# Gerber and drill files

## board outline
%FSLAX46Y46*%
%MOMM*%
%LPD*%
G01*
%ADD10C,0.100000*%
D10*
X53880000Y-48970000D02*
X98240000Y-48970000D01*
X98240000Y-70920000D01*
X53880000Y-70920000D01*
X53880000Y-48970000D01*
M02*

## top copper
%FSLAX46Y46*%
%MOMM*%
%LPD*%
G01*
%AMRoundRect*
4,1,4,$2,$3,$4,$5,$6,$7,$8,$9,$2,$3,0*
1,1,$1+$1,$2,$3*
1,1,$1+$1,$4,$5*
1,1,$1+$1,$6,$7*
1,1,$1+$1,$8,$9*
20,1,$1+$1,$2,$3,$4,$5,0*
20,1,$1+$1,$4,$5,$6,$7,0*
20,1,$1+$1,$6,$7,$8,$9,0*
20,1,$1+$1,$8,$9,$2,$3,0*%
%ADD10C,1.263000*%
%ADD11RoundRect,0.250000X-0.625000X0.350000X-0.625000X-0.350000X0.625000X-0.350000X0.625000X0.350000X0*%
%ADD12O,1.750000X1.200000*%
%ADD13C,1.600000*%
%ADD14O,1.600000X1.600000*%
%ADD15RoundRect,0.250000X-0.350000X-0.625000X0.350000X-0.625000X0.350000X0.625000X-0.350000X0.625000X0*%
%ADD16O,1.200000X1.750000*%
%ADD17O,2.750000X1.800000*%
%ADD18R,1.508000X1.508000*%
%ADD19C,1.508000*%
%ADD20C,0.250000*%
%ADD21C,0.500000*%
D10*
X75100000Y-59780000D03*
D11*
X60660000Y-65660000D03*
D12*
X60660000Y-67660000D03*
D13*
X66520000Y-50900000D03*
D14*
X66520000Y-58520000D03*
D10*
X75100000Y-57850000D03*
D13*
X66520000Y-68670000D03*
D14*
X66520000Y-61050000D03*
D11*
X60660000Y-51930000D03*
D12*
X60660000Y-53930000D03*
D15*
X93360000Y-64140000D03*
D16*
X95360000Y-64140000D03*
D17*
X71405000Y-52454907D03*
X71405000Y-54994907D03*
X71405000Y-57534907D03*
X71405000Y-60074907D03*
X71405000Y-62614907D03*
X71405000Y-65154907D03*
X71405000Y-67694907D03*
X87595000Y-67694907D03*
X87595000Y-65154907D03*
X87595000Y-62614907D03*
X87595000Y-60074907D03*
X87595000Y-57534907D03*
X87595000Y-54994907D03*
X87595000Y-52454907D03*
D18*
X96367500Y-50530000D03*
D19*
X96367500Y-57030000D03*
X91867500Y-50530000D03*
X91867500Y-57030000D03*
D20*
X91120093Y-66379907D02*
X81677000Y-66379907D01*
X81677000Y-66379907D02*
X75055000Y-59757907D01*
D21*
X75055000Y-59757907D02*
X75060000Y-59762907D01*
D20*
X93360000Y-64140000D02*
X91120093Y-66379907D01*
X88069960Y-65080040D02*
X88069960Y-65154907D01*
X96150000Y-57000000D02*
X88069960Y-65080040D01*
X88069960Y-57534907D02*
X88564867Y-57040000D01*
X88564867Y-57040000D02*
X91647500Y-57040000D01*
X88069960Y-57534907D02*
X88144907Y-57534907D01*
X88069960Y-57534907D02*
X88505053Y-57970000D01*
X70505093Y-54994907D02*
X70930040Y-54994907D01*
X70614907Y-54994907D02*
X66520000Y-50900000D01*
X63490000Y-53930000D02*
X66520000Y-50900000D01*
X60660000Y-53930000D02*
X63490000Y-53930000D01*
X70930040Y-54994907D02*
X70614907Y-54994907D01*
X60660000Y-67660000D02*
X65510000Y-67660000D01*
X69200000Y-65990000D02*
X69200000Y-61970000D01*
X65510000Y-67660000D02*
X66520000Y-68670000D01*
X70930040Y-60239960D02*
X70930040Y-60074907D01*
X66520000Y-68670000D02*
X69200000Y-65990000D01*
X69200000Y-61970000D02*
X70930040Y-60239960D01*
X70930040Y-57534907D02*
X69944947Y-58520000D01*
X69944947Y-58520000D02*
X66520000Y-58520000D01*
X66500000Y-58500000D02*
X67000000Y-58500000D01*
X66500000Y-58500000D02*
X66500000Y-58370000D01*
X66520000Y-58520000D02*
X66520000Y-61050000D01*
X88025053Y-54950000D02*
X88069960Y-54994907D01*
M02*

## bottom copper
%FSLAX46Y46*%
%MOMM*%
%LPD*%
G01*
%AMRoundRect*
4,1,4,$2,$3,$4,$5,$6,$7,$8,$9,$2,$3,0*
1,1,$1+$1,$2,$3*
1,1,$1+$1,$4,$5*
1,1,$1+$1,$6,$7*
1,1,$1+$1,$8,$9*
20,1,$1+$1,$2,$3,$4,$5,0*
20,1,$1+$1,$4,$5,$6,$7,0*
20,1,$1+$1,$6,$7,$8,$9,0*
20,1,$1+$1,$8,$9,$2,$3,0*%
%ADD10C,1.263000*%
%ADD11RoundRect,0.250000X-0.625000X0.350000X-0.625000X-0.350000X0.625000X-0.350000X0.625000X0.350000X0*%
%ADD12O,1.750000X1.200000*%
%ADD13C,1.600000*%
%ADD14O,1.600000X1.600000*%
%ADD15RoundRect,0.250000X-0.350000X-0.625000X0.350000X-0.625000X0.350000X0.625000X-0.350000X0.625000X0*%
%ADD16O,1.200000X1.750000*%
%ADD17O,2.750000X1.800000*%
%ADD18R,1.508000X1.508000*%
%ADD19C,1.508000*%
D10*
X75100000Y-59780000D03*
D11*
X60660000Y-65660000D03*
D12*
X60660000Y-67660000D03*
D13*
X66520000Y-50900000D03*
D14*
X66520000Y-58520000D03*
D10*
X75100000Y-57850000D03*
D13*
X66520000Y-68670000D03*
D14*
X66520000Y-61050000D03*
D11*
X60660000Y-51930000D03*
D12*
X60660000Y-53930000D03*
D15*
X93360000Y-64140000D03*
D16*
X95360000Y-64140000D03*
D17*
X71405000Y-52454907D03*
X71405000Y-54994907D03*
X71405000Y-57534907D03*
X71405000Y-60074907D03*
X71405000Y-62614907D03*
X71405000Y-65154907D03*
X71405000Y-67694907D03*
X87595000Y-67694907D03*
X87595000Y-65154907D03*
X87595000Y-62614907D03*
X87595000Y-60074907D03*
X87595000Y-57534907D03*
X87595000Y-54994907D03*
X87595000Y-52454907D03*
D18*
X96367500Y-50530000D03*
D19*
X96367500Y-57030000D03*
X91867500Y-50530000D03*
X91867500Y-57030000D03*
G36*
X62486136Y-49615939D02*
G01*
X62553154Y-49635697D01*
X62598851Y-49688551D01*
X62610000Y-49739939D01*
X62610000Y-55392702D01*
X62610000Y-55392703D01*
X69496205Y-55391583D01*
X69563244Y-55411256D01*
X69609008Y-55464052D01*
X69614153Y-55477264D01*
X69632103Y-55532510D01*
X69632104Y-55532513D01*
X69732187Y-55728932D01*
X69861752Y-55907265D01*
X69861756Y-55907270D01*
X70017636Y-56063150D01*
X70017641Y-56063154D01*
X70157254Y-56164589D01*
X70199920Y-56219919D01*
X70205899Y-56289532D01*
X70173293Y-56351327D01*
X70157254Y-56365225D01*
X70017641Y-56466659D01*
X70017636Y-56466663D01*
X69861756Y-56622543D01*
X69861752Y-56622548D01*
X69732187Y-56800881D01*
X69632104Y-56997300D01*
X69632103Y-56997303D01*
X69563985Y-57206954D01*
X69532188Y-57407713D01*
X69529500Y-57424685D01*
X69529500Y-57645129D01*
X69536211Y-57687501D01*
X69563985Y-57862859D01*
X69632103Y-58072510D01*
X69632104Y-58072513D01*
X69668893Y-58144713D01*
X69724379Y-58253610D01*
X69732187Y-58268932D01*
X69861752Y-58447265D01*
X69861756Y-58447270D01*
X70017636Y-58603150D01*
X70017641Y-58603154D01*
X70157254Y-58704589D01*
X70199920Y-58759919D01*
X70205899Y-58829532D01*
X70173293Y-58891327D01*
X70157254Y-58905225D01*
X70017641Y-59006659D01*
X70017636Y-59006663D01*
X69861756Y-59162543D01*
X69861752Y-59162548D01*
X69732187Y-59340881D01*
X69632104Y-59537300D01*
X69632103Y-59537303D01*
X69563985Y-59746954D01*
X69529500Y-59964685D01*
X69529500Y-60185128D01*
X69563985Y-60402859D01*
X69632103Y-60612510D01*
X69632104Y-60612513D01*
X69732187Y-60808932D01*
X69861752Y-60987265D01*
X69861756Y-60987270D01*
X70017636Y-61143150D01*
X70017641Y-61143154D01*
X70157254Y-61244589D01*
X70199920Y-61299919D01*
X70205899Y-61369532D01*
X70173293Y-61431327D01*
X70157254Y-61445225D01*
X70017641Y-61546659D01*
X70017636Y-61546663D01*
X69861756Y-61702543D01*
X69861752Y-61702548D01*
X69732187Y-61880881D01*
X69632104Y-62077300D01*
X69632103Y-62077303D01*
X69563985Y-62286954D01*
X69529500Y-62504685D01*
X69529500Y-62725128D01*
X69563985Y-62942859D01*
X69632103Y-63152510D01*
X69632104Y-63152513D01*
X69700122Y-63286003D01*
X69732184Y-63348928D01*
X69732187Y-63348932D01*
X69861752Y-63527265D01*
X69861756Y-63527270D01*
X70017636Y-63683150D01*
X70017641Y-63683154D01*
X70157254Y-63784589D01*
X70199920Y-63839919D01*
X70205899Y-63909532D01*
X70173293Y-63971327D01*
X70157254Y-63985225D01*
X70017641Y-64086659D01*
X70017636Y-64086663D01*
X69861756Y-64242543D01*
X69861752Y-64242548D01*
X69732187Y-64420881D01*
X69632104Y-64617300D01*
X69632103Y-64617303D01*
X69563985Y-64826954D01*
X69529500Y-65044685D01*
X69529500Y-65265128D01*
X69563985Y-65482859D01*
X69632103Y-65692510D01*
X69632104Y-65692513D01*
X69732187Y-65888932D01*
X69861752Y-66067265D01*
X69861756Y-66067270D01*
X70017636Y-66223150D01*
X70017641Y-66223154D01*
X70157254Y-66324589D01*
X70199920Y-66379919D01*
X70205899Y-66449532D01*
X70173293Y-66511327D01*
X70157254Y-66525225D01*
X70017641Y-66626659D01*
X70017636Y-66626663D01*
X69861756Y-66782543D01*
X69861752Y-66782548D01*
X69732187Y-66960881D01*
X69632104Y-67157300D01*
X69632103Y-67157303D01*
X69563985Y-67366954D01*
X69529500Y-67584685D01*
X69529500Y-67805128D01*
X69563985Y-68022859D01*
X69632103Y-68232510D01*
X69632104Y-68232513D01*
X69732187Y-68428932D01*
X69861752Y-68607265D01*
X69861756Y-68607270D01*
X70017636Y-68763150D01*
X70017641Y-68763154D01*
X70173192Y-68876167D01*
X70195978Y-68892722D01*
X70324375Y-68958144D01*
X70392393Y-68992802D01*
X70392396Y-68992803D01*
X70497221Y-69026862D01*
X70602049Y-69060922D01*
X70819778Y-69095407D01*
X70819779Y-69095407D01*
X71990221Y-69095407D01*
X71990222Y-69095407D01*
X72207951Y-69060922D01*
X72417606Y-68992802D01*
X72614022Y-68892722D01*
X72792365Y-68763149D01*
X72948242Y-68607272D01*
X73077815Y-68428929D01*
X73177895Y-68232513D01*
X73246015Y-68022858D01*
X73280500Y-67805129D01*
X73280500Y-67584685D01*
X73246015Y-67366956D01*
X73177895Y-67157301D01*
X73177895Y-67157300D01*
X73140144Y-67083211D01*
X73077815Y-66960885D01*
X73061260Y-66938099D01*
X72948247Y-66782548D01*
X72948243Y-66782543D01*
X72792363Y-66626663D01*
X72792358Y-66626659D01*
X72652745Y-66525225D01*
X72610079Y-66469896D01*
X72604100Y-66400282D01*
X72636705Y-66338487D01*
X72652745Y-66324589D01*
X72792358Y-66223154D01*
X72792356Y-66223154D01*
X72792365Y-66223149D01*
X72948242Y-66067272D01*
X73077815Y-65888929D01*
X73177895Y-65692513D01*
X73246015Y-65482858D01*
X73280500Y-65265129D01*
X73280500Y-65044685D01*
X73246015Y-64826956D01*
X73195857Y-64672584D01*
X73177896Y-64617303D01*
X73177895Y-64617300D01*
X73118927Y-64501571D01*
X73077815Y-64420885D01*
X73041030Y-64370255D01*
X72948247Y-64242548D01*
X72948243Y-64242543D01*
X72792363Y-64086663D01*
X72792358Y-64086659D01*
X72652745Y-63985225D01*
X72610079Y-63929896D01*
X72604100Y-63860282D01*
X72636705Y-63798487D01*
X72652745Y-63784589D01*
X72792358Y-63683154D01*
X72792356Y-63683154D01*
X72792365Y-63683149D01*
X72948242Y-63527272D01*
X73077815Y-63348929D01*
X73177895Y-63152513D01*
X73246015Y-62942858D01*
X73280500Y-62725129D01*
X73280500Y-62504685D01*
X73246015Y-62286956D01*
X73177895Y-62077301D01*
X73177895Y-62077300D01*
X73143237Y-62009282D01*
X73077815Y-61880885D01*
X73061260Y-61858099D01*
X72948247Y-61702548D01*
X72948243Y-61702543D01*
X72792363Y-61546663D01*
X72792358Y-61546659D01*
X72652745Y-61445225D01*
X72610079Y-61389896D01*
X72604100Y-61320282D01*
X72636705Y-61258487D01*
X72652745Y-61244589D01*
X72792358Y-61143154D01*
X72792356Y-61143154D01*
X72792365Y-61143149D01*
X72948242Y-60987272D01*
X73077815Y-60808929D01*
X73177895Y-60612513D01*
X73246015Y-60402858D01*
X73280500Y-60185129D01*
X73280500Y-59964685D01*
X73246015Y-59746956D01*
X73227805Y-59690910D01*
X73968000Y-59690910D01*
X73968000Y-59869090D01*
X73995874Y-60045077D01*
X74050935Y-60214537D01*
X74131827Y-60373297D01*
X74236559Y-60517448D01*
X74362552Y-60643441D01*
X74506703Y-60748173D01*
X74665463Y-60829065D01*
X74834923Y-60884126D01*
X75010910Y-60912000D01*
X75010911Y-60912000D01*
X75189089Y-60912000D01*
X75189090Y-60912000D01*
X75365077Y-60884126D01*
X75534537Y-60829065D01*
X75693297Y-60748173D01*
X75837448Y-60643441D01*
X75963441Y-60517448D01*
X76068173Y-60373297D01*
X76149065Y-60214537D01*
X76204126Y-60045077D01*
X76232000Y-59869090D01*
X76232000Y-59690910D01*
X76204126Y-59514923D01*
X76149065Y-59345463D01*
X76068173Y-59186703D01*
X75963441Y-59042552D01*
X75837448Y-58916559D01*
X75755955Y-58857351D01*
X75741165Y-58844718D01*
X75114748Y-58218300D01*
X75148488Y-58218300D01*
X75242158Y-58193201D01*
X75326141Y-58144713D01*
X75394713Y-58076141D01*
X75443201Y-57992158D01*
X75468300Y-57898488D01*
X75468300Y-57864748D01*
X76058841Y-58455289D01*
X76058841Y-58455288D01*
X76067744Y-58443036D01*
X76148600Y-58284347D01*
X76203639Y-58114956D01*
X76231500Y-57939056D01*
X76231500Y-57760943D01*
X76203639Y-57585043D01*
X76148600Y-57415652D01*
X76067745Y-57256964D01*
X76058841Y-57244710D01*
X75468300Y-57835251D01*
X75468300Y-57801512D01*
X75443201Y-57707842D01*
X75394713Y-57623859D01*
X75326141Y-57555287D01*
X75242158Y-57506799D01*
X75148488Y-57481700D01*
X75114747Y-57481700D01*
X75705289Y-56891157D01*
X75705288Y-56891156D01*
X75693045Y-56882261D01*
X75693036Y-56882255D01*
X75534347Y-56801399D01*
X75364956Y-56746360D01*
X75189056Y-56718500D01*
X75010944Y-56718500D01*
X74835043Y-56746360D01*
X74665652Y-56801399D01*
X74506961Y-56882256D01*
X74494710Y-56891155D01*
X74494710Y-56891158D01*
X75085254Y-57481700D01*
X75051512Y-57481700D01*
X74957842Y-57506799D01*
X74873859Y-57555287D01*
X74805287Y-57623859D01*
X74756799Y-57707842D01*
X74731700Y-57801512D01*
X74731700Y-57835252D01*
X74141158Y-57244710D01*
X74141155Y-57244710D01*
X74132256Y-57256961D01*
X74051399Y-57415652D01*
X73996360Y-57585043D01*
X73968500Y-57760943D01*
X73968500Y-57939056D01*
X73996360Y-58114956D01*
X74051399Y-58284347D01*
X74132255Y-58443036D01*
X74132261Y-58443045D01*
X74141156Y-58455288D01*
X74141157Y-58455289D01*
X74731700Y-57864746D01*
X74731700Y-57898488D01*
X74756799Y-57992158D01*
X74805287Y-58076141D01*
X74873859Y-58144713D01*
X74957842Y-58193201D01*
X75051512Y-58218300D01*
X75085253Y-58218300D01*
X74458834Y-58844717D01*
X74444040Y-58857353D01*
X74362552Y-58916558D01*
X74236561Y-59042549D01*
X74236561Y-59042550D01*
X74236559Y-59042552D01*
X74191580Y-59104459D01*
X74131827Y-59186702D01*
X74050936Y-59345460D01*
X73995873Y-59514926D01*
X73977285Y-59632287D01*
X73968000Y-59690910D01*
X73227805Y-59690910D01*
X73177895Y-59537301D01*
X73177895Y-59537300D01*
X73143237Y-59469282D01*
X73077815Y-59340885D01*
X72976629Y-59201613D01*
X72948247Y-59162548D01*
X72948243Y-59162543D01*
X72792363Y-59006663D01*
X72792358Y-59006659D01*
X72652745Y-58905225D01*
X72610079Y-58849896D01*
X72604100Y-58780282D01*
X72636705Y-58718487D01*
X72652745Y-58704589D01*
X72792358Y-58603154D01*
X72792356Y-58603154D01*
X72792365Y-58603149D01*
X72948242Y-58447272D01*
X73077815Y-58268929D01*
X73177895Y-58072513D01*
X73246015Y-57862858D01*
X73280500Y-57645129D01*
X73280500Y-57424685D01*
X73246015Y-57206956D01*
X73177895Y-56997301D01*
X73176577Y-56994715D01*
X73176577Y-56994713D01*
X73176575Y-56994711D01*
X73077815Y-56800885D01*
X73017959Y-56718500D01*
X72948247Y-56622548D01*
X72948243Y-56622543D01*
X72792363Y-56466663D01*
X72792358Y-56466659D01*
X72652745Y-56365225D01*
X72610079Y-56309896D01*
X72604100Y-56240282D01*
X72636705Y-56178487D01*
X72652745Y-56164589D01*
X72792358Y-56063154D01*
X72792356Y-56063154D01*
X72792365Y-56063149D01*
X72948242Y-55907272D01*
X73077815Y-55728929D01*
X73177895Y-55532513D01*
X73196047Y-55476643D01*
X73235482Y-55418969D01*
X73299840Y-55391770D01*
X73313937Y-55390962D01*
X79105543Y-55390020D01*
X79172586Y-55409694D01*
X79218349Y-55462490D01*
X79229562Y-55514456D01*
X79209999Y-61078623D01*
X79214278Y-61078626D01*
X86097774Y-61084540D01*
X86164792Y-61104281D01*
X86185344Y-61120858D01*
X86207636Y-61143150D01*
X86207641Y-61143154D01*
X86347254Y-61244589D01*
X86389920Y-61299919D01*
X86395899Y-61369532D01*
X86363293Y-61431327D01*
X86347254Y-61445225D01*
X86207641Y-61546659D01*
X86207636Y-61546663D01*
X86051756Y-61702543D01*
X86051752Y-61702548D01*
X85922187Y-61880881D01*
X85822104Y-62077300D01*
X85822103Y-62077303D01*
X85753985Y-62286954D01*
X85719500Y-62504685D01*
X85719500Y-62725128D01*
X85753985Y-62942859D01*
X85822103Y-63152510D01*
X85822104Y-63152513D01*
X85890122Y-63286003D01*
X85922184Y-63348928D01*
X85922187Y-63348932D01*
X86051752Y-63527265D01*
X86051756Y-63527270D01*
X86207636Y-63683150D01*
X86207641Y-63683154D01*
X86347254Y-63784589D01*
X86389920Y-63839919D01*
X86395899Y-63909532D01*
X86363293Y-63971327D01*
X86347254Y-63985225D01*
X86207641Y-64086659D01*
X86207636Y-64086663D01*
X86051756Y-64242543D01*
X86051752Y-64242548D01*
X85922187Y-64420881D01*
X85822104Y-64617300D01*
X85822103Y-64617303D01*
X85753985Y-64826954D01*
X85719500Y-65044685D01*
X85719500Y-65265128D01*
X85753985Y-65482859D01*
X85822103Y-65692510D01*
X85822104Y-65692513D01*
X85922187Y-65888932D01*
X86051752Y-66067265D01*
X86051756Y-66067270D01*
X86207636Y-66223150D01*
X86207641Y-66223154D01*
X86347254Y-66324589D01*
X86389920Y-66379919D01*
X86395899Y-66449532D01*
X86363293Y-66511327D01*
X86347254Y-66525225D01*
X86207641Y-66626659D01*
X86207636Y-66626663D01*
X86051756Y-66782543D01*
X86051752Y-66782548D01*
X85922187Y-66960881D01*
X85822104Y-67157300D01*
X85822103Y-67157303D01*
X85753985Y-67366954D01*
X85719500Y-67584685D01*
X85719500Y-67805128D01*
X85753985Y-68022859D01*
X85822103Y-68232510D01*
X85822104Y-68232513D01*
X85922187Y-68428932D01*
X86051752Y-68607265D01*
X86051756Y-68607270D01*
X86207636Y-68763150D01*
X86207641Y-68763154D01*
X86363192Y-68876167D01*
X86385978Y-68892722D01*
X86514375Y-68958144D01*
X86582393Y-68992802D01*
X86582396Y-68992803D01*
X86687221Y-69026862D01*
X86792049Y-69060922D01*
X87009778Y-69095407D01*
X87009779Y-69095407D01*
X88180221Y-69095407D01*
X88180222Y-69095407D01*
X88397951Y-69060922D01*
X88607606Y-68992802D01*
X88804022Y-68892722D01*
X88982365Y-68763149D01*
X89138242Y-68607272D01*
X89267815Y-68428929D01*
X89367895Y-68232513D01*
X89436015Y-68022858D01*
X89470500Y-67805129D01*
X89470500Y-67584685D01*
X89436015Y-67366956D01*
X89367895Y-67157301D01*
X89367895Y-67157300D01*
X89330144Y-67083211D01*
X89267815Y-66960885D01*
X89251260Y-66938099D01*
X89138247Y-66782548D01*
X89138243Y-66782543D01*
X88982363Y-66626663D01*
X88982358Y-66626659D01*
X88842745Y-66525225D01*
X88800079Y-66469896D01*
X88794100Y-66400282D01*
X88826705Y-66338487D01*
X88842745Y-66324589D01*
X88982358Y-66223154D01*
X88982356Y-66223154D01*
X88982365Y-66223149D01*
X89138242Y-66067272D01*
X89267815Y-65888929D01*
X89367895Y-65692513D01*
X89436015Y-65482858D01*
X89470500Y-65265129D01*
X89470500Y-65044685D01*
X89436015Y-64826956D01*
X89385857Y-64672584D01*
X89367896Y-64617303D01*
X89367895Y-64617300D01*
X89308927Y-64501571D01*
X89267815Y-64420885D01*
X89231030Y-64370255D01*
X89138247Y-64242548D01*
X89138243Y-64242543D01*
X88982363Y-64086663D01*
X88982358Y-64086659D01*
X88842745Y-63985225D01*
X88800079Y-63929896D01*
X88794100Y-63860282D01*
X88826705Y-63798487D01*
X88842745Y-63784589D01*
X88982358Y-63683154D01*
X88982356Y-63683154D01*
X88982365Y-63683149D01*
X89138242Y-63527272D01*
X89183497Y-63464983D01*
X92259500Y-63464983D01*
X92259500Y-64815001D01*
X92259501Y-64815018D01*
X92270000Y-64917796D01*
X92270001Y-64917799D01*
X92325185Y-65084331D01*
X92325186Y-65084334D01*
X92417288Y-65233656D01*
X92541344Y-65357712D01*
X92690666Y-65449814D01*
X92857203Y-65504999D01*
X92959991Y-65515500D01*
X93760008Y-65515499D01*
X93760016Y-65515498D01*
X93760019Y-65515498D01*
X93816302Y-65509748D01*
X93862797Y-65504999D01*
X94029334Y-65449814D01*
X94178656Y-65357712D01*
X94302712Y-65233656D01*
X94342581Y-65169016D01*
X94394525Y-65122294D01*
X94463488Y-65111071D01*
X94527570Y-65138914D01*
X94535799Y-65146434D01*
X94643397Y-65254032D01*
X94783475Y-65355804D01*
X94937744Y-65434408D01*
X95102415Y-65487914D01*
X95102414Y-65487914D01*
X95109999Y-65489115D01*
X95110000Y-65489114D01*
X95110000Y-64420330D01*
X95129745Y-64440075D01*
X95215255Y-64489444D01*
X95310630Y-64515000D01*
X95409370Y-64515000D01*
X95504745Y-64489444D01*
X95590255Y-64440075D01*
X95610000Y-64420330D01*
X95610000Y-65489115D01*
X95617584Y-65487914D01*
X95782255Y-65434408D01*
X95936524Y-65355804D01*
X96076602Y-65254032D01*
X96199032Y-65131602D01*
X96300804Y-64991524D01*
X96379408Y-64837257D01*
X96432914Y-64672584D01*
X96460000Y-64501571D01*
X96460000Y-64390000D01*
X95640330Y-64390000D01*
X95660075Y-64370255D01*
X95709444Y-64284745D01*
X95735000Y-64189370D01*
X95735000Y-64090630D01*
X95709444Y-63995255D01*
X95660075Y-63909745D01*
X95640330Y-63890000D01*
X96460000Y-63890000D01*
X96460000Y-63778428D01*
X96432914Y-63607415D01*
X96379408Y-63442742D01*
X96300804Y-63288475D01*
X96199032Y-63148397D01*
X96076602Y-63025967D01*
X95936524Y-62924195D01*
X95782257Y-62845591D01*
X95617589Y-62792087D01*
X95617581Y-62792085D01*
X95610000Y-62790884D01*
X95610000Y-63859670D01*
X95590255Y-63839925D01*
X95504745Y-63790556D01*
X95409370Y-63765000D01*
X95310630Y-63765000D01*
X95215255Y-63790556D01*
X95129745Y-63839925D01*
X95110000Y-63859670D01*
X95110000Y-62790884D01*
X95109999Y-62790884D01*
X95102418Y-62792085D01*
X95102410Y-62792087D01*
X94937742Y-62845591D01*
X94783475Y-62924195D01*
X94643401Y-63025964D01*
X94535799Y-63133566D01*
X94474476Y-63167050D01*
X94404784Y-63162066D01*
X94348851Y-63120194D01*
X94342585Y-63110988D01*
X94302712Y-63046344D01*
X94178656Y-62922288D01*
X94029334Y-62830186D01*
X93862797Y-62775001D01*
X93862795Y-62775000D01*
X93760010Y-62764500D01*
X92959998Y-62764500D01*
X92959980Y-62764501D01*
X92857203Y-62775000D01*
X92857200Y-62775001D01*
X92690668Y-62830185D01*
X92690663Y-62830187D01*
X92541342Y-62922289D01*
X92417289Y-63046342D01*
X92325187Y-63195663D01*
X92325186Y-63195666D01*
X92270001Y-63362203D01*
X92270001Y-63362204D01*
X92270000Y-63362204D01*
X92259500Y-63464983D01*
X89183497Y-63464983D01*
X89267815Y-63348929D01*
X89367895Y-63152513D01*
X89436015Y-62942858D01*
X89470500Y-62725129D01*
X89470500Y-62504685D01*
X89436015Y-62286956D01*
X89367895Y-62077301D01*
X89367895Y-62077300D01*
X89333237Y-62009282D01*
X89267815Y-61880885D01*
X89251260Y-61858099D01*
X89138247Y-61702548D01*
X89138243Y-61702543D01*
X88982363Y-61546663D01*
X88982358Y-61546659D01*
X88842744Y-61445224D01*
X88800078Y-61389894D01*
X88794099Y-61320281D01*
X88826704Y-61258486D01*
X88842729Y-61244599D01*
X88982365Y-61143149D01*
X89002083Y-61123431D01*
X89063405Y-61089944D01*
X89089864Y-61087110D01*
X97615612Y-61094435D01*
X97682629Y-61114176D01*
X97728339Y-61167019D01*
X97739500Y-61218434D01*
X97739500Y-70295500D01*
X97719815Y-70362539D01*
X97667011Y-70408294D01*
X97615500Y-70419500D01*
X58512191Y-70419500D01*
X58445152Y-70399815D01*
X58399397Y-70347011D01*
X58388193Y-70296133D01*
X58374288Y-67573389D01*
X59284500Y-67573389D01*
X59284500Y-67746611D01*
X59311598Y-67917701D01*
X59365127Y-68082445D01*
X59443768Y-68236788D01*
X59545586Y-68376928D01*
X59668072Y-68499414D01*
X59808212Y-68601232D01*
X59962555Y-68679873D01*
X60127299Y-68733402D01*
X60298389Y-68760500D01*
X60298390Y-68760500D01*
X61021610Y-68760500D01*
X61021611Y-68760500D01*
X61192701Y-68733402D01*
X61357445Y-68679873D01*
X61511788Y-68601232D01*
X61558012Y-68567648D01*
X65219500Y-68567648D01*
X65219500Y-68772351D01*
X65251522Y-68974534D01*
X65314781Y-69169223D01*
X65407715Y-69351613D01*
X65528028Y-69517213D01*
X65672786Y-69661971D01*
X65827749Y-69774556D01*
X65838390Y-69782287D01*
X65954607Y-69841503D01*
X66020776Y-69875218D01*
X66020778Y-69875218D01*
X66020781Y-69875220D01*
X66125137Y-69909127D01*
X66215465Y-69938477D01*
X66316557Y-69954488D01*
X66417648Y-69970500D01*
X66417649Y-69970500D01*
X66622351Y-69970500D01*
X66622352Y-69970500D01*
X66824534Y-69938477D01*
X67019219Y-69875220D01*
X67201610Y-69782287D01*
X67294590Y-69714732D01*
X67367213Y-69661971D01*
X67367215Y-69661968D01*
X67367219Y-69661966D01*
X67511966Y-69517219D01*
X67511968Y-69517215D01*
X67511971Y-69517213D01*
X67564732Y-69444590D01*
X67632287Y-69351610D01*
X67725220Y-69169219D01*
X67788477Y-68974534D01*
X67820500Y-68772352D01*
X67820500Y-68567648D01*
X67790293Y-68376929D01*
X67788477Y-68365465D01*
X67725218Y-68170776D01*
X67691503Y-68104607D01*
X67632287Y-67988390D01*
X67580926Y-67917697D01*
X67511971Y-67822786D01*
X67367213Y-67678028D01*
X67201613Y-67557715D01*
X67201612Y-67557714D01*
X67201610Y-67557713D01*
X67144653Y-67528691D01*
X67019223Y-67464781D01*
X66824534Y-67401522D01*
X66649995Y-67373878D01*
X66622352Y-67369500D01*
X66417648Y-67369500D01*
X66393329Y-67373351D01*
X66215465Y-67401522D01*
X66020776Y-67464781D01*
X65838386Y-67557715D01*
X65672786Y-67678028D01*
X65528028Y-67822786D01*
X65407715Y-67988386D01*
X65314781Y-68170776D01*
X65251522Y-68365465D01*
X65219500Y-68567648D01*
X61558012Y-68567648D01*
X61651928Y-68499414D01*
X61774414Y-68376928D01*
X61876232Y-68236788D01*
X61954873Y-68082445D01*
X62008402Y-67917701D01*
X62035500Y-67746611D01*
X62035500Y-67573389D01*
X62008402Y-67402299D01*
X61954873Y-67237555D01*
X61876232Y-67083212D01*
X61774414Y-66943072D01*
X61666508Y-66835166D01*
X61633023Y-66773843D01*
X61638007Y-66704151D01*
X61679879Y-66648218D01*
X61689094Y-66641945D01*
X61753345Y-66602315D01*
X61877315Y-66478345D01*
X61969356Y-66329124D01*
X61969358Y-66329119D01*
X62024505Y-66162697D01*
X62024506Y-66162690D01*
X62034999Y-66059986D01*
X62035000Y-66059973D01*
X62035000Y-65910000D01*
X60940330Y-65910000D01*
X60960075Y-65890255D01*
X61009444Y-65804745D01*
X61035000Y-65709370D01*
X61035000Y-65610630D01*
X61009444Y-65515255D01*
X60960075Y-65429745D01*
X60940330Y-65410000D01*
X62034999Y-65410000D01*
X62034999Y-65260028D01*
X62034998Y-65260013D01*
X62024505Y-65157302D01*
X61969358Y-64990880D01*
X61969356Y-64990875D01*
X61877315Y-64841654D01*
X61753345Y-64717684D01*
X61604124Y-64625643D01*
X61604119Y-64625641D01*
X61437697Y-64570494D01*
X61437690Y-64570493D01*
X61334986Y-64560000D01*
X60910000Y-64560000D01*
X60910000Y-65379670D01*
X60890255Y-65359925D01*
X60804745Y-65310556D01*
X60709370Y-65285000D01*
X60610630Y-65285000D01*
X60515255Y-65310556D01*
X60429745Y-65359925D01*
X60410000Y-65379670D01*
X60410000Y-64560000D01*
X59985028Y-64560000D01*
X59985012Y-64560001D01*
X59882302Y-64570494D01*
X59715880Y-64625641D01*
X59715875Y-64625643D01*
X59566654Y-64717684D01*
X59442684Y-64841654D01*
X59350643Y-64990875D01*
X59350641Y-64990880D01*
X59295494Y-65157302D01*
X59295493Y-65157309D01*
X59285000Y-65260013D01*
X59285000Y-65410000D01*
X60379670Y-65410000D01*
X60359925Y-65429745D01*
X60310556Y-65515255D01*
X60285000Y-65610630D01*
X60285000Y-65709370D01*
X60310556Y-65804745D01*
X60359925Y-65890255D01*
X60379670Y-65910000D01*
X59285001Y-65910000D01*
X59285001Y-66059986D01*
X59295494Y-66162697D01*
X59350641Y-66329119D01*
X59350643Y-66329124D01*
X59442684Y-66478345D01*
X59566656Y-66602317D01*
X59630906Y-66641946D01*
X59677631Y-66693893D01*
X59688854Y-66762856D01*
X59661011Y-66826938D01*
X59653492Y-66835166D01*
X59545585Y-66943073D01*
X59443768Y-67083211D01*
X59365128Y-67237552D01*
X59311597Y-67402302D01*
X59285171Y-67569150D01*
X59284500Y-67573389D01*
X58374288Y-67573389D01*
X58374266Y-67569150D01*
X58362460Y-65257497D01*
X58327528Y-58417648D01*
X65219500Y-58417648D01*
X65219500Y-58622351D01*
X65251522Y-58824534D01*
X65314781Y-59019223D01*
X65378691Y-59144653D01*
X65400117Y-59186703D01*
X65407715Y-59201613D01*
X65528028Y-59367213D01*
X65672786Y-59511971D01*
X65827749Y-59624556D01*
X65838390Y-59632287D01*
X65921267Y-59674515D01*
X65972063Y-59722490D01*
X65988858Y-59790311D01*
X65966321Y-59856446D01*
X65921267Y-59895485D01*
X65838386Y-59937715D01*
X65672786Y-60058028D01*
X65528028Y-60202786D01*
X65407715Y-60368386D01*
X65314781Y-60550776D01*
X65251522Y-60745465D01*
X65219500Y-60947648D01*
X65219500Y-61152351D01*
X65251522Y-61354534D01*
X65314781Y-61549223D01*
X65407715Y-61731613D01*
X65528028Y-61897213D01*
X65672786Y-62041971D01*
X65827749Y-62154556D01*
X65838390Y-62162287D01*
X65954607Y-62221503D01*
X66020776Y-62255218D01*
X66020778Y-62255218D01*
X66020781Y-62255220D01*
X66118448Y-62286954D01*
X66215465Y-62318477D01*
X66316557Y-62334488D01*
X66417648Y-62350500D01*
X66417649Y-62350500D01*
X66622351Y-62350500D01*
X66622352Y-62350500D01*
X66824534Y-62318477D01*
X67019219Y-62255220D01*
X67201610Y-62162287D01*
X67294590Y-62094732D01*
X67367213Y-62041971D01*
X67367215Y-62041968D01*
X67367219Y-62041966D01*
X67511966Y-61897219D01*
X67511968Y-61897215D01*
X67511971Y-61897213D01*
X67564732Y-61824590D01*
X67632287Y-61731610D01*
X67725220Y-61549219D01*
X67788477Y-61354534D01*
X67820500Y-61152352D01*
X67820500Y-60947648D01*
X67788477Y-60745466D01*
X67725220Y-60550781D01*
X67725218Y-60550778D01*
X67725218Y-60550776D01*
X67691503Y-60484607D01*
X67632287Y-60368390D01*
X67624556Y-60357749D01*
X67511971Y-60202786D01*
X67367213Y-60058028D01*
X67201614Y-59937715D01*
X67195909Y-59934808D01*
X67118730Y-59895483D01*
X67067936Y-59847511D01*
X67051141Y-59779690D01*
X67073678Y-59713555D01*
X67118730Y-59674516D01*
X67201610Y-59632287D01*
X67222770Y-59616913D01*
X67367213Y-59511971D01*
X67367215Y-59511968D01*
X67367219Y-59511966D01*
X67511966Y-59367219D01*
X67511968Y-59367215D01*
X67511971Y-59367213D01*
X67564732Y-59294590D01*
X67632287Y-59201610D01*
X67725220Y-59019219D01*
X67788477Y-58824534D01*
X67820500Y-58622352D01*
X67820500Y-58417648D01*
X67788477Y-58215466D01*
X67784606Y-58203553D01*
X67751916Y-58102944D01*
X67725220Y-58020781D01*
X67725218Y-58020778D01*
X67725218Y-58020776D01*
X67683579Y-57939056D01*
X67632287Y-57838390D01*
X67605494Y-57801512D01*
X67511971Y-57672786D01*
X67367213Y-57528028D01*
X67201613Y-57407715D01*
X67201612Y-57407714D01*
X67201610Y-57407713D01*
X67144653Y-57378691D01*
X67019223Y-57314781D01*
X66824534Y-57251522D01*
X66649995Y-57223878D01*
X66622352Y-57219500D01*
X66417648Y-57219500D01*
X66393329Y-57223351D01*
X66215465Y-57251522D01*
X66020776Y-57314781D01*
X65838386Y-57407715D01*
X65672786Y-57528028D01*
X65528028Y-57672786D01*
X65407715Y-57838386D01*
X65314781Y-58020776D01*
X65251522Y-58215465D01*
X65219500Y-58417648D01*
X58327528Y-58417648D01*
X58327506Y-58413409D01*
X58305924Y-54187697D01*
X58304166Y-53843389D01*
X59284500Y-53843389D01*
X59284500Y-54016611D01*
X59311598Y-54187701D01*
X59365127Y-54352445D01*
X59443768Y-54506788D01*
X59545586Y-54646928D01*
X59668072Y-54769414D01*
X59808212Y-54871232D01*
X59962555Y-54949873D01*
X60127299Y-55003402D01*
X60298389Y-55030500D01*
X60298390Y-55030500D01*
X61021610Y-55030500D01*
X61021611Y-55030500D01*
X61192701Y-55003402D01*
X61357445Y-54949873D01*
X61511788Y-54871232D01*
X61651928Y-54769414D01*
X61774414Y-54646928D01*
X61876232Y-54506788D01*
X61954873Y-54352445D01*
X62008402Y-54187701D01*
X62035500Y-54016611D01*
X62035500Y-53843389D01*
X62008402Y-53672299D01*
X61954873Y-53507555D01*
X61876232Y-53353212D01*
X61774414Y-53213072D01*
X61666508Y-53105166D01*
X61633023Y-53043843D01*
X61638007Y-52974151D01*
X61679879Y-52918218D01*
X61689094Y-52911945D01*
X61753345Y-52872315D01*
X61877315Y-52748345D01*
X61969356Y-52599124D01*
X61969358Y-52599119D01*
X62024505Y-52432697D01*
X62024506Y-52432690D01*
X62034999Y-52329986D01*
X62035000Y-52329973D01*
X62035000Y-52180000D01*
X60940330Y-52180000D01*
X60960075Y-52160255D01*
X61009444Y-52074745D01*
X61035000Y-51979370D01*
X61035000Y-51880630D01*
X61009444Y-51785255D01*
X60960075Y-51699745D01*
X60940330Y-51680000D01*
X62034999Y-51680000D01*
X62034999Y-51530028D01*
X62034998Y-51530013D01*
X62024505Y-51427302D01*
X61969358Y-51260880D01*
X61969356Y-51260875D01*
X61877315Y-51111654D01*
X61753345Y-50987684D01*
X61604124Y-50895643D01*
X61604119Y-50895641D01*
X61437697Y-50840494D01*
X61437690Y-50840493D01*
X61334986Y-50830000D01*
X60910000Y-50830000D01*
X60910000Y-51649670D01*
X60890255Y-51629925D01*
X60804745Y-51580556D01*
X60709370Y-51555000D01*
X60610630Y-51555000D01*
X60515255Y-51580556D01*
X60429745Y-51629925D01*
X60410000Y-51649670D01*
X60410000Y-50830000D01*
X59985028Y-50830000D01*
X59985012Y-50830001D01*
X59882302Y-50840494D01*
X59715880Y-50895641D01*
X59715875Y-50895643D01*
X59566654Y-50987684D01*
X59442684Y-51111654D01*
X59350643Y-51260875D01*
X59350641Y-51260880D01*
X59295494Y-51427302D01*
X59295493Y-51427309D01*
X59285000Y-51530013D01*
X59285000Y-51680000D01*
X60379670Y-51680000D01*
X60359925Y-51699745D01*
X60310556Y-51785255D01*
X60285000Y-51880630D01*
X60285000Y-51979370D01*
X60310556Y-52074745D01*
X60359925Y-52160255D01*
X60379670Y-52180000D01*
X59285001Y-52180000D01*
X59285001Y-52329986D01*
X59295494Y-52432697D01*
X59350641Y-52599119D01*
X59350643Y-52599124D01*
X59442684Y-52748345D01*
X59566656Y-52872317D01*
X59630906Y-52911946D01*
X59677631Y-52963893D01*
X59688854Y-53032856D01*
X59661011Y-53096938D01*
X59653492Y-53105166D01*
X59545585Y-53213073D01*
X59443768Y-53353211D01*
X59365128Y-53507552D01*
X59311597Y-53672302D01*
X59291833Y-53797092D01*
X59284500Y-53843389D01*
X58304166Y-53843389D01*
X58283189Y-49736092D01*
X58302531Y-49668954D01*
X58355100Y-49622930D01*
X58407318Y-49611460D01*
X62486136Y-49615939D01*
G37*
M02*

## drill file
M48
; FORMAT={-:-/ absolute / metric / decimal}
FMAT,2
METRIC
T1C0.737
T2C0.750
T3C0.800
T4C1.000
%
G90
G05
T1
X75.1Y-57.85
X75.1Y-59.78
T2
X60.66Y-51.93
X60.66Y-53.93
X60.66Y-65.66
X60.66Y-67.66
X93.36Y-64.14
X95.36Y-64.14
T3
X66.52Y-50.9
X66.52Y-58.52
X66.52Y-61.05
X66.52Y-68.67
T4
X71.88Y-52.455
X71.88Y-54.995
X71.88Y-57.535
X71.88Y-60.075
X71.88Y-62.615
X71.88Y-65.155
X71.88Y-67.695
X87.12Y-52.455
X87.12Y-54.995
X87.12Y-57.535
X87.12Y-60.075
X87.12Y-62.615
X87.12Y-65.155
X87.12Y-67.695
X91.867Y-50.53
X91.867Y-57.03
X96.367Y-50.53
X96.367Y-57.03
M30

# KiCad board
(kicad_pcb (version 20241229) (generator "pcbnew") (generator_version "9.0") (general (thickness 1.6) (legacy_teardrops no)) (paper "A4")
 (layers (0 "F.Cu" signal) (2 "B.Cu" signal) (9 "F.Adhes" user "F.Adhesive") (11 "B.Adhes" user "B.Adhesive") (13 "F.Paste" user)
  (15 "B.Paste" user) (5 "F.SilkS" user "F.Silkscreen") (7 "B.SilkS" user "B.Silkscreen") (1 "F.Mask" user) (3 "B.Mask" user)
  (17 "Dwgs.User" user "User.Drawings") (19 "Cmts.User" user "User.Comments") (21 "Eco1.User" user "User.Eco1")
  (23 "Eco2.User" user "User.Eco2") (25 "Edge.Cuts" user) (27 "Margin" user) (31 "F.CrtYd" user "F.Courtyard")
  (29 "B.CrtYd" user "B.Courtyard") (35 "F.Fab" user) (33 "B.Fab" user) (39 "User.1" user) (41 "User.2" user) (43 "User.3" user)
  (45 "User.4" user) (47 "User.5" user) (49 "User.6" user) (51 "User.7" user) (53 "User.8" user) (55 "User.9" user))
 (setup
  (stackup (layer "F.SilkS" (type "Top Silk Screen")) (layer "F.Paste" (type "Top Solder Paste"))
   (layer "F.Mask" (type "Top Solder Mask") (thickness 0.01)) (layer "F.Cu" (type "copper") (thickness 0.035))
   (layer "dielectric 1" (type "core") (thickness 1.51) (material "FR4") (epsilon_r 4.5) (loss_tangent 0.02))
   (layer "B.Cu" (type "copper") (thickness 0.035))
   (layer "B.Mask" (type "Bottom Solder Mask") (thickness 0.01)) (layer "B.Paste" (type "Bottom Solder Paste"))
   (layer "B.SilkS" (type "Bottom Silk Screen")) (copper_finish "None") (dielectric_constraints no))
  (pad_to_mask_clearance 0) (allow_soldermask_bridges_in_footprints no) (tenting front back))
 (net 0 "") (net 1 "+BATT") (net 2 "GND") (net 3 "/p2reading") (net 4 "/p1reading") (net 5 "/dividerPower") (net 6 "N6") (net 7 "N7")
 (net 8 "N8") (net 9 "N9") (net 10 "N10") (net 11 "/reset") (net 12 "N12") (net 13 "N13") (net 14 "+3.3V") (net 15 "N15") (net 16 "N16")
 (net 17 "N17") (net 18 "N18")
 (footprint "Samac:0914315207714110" (layer "F.Cu") (at 75.1 59.78)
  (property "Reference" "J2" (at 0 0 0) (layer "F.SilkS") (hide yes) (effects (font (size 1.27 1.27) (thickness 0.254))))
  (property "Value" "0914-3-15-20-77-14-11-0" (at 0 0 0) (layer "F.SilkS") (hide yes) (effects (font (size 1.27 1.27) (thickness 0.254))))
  (pad "1" thru_hole circle (at 0 0) (size 1.263 1.263) (drill 0.7366) (layers "*.Cu" "*.Mask") (remove_unused_layers no) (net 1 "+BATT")))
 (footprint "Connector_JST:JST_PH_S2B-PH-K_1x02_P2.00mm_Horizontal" (layer "F.Cu") (at 60.66 65.66 -90)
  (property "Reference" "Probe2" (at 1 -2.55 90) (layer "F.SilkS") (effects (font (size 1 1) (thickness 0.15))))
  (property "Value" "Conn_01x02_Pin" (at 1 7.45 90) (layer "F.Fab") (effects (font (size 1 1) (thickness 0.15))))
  (pad "1" thru_hole roundrect (at 0 0 270) (size 1.2 1.75) (drill 0.75) (layers "*.Cu" "*.Mask") (remove_unused_layers no)
   (roundrect_rratio 0.208333) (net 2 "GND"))
  (pad "2" thru_hole oval (at 2 0 270) (size 1.2 1.75) (drill 0.75) (layers "*.Cu" "*.Mask") (remove_unused_layers no) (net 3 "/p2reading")))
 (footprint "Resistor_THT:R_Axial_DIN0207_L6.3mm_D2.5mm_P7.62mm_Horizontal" (layer "F.Cu") (at 66.52 50.9 -90)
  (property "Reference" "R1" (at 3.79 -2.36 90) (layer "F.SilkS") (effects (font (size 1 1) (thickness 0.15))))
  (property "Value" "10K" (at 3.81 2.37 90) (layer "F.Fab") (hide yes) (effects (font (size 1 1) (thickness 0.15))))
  (pad "1" thru_hole circle (at 0 0 270) (size 1.6 1.6) (drill 0.8) (layers "*.Cu" "*.Mask") (remove_unused_layers no) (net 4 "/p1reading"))
  (pad "2" thru_hole oval (at 7.62 0 270) (size 1.6 1.6) (drill 0.8) (layers "*.Cu" "*.Mask") (remove_unused_layers no)
   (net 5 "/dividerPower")))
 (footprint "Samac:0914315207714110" (layer "F.Cu") (at 75.1 57.85)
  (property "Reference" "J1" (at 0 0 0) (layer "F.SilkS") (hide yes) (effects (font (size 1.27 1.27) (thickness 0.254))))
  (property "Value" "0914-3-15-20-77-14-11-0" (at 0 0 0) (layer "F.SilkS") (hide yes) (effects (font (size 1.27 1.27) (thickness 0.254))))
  (pad "1" thru_hole circle (at 0 0) (size 1.263 1.263) (drill 0.7366) (layers "*.Cu" "*.Mask") (remove_unused_layers no) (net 2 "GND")))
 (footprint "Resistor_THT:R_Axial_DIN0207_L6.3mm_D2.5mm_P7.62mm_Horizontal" (layer "F.Cu") (at 66.52 68.67 90)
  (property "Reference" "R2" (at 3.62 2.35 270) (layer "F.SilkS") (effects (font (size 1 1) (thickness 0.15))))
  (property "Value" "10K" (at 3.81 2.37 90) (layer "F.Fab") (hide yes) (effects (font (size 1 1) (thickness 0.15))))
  (pad "1" thru_hole circle (at 0 0 90) (size 1.6 1.6) (drill 0.8) (layers "*.Cu" "*.Mask") (remove_unused_layers no) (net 3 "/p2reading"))
  (pad "2" thru_hole oval (at 7.62 0 90) (size 1.6 1.6) (drill 0.8) (layers "*.Cu" "*.Mask") (remove_unused_layers no)
   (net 5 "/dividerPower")))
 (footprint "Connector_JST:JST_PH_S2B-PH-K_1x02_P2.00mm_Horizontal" (layer "F.Cu") (at 60.66 51.93 -90)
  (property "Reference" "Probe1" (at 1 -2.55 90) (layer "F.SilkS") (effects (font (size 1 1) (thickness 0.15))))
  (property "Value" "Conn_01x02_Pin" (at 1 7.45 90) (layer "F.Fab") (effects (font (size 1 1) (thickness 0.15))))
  (pad "1" thru_hole roundrect (at 0 0 270) (size 1.2 1.75) (drill 0.75) (layers "*.Cu" "*.Mask") (remove_unused_layers no)
   (roundrect_rratio 0.208333) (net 2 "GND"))
  (pad "2" thru_hole oval (at 2 0 270) (size 1.2 1.75) (drill 0.75) (layers "*.Cu" "*.Mask") (remove_unused_layers no) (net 4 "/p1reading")))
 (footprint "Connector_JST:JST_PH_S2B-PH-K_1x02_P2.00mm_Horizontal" (layer "F.Cu") (at 93.36 64.14)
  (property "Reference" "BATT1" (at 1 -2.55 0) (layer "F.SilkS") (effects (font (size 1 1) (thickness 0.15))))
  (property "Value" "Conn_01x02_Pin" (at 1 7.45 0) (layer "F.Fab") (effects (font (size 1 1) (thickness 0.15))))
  (pad "1" thru_hole roundrect (at 0 0) (size 1.2 1.75) (drill 0.75) (layers "*.Cu" "*.Mask") (remove_unused_layers no)
   (roundrect_rratio 0.208333) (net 1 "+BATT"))
  (pad "2" thru_hole oval (at 2 0) (size 1.2 1.75) (drill 0.75) (layers "*.Cu" "*.Mask") (remove_unused_layers no) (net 2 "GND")))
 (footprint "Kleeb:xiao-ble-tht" (layer "F.Cu") (at 79.5 60.074907)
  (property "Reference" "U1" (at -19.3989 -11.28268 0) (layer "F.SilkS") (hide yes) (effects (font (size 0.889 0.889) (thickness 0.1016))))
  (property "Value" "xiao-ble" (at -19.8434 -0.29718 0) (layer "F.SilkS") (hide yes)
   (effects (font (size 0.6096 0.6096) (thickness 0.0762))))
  (pad "1" thru_hole oval (at -7.62 -7.62) (size 2.75 1.8) (drill 1 (offset -0.475 0)) (layers "*.Cu" "*.Mask") (remove_unused_layers no)
   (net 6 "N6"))
  (pad "2" thru_hole oval (at -7.62 -5.08) (size 2.75 1.8) (drill 1 (offset -0.475 0)) (layers "*.Cu" "*.Mask") (remove_unused_layers no)
   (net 4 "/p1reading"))
  (pad "3" thru_hole oval (at -7.62 -2.54) (size 2.75 1.8) (drill 1 (offset -0.475 0)) (layers "*.Cu" "*.Mask") (remove_unused_layers no)
   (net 5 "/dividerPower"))
  (pad "4" thru_hole oval (at -7.62 0) (size 2.75 1.8) (drill 1 (offset -0.475 0)) (layers "*.Cu" "*.Mask") (remove_unused_layers no)
   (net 3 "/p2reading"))
  (pad "5" thru_hole oval (at -7.62 2.54) (size 2.75 1.8) (drill 1 (offset -0.475 0)) (layers "*.Cu" "*.Mask") (remove_unused_layers no)
   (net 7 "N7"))
  (pad "6" thru_hole oval (at -7.62 5.08) (size 2.75 1.8) (drill 1 (offset -0.475 0)) (layers "*.Cu" "*.Mask") (remove_unused_layers no)
   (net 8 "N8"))
  (pad "7" thru_hole oval (at -7.62 7.62) (size 2.75 1.8) (drill 1 (offset -0.475 0)) (layers "*.Cu" "*.Mask") (remove_unused_layers no)
   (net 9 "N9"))
  (pad "8" thru_hole oval (at 7.62 7.62 180) (size 2.75 1.8) (drill 1 (offset -0.475 0)) (layers "*.Cu" "*.Mask") (remove_unused_layers no)
   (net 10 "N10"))
  (pad "9" thru_hole oval (at 7.62 5.08 180) (size 2.75 1.8) (drill 1 (offset -0.475 0)) (layers "*.Cu" "*.Mask") (remove_unused_layers no)
   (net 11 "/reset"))
  (pad "10" thru_hole oval (at 7.62 2.54 180) (size 2.75 1.8) (drill 1 (offset -0.475 0)) (layers "*.Cu" "*.Mask") (remove_unused_layers no)
   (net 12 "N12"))
  (pad "11" thru_hole oval (at 7.62 0 180) (size 2.75 1.8) (drill 1 (offset -0.475 0)) (layers "*.Cu" "*.Mask") (remove_unused_layers no)
   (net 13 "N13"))
  (pad "12" thru_hole oval (at 7.62 -2.54 180) (size 2.75 1.8) (drill 1 (offset -0.475 0)) (layers "*.Cu" "*.Mask")
   (remove_unused_layers no) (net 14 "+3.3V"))
  (pad "13" thru_hole oval (at 7.62 -5.08 180) (size 2.75 1.8) (drill 1 (offset -0.475 0)) (layers "*.Cu" "*.Mask")
   (remove_unused_layers no) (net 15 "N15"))
  (pad "14" thru_hole oval (at 7.62 -7.62 180) (size 2.75 1.8) (drill 1 (offset -0.475 0)) (layers "*.Cu" "*.Mask")
   (remove_unused_layers no) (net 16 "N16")))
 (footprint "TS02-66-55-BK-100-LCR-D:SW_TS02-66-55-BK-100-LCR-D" (layer "F.Cu") (at 94.1175 53.78 -90)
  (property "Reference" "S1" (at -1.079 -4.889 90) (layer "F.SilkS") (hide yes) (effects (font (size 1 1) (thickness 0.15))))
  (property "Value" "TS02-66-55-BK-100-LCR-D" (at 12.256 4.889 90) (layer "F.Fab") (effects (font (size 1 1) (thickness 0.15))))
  (pad "1" thru_hole rect (at -3.25 -2.25 270) (size 1.508 1.508) (drill 1) (layers "*.Cu" "*.Mask") (remove_unused_layers no)
   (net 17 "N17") (solder_mask_margin 0.102))
  (pad "2" thru_hole circle (at 3.25 -2.25 270) (size 1.508 1.508) (drill 1) (layers "*.Cu" "*.Mask") (remove_unused_layers no)
   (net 11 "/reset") (solder_mask_margin 0.102))
  (pad "3" thru_hole circle (at -3.25 2.25 270) (size 1.508 1.508) (drill 1) (layers "*.Cu" "*.Mask") (remove_unused_layers no)
   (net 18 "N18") (solder_mask_margin 0.102))
  (pad "4" thru_hole circle (at 3.25 2.25 270) (size 1.508 1.508) (drill 1) (layers "*.Cu" "*.Mask") (remove_unused_layers no)
   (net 14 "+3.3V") (solder_mask_margin 0.102)))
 (gr_rect (start 53.88 48.97) (end 98.24 70.92) (stroke (width 0.1) (type default)) (fill no) (layer "Edge.Cuts"))
 (segment (start 91.120093 66.379907) (end 81.677 66.379907) (width 0.25) (layer "F.Cu") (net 1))
 (segment (start 81.677 66.379907) (end 75.055 59.757907) (width 0.25) (layer "F.Cu") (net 1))
 (segment (start 75.055 59.757907) (end 75.06 59.762907) (width 0.5) (layer "F.Cu") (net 1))
 (segment (start 93.36 64.14) (end 91.120093 66.379907) (width 0.25) (layer "F.Cu") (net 1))
 (segment (start 88.06996 65.08004) (end 88.06996 65.154907) (width 0.25) (layer "F.Cu") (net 11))
 (segment (start 96.15 57) (end 88.06996 65.08004) (width 0.25) (layer "F.Cu") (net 11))
 (segment (start 88.06996 57.534907) (end 88.564867 57.04) (width 0.25) (layer "F.Cu") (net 14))
 (segment (start 88.564867 57.04) (end 91.6475 57.04) (width 0.25) (layer "F.Cu") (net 14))
 (segment (start 88.06996 57.534907) (end 88.144907 57.534907) (width 0.25) (layer "F.Cu") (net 14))
 (segment (start 88.06996 57.534907) (end 88.505053 57.97) (width 0.25) (layer "F.Cu") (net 14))
 (segment (start 70.505093 54.994907) (end 70.93004 54.994907) (width 0.25) (layer "F.Cu") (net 4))
 (segment (start 70.614907 54.994907) (end 66.52 50.9) (width 0.25) (layer "F.Cu") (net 4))
 (segment (start 63.49 53.93) (end 66.52 50.9) (width 0.25) (layer "F.Cu") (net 4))
 (segment (start 60.66 53.93) (end 63.49 53.93) (width 0.25) (layer "F.Cu") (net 4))
 (segment (start 70.93004 54.994907) (end 70.614907 54.994907) (width 0.25) (layer "F.Cu") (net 4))
 (segment (start 60.66 67.66) (end 65.51 67.66) (width 0.25) (layer "F.Cu") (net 3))
 (segment (start 69.2 65.99) (end 69.2 61.97) (width 0.25) (layer "F.Cu") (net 3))
 (segment (start 65.51 67.66) (end 66.52 68.67) (width 0.25) (layer "F.Cu") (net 3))
 (segment (start 70.93004 60.23996) (end 70.93004 60.074907) (width 0.25) (layer "F.Cu") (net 3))
 (segment (start 66.52 68.67) (end 69.2 65.99) (width 0.25) (layer "F.Cu") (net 3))
 (segment (start 69.2 61.97) (end 70.93004 60.23996) (width 0.25) (layer "F.Cu") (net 3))
 (segment (start 70.93004 57.534907) (end 69.944947 58.52) (width 0.25) (layer "F.Cu") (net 5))
 (segment (start 69.944947 58.52) (end 66.52 58.52) (width 0.25) (layer "F.Cu") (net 5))
 (segment (start 66.5 58.5) (end 67 58.5) (width 0.25) (layer "F.Cu") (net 5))
 (segment (start 66.5 58.5) (end 66.5 58.37) (width 0.25) (layer "F.Cu") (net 5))
 (segment (start 66.52 58.52) (end 66.52 61.05) (width 0.25) (layer "F.Cu") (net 5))
 (segment (start 88.025053 54.95) (end 88.06996 54.994907) (width 0.25) (layer "F.Cu") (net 15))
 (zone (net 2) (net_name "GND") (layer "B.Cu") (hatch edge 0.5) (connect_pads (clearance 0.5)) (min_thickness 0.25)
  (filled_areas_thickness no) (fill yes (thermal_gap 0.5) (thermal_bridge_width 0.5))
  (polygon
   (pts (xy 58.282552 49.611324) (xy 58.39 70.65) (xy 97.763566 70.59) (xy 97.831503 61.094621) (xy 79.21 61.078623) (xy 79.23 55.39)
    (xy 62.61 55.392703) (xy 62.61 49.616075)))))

